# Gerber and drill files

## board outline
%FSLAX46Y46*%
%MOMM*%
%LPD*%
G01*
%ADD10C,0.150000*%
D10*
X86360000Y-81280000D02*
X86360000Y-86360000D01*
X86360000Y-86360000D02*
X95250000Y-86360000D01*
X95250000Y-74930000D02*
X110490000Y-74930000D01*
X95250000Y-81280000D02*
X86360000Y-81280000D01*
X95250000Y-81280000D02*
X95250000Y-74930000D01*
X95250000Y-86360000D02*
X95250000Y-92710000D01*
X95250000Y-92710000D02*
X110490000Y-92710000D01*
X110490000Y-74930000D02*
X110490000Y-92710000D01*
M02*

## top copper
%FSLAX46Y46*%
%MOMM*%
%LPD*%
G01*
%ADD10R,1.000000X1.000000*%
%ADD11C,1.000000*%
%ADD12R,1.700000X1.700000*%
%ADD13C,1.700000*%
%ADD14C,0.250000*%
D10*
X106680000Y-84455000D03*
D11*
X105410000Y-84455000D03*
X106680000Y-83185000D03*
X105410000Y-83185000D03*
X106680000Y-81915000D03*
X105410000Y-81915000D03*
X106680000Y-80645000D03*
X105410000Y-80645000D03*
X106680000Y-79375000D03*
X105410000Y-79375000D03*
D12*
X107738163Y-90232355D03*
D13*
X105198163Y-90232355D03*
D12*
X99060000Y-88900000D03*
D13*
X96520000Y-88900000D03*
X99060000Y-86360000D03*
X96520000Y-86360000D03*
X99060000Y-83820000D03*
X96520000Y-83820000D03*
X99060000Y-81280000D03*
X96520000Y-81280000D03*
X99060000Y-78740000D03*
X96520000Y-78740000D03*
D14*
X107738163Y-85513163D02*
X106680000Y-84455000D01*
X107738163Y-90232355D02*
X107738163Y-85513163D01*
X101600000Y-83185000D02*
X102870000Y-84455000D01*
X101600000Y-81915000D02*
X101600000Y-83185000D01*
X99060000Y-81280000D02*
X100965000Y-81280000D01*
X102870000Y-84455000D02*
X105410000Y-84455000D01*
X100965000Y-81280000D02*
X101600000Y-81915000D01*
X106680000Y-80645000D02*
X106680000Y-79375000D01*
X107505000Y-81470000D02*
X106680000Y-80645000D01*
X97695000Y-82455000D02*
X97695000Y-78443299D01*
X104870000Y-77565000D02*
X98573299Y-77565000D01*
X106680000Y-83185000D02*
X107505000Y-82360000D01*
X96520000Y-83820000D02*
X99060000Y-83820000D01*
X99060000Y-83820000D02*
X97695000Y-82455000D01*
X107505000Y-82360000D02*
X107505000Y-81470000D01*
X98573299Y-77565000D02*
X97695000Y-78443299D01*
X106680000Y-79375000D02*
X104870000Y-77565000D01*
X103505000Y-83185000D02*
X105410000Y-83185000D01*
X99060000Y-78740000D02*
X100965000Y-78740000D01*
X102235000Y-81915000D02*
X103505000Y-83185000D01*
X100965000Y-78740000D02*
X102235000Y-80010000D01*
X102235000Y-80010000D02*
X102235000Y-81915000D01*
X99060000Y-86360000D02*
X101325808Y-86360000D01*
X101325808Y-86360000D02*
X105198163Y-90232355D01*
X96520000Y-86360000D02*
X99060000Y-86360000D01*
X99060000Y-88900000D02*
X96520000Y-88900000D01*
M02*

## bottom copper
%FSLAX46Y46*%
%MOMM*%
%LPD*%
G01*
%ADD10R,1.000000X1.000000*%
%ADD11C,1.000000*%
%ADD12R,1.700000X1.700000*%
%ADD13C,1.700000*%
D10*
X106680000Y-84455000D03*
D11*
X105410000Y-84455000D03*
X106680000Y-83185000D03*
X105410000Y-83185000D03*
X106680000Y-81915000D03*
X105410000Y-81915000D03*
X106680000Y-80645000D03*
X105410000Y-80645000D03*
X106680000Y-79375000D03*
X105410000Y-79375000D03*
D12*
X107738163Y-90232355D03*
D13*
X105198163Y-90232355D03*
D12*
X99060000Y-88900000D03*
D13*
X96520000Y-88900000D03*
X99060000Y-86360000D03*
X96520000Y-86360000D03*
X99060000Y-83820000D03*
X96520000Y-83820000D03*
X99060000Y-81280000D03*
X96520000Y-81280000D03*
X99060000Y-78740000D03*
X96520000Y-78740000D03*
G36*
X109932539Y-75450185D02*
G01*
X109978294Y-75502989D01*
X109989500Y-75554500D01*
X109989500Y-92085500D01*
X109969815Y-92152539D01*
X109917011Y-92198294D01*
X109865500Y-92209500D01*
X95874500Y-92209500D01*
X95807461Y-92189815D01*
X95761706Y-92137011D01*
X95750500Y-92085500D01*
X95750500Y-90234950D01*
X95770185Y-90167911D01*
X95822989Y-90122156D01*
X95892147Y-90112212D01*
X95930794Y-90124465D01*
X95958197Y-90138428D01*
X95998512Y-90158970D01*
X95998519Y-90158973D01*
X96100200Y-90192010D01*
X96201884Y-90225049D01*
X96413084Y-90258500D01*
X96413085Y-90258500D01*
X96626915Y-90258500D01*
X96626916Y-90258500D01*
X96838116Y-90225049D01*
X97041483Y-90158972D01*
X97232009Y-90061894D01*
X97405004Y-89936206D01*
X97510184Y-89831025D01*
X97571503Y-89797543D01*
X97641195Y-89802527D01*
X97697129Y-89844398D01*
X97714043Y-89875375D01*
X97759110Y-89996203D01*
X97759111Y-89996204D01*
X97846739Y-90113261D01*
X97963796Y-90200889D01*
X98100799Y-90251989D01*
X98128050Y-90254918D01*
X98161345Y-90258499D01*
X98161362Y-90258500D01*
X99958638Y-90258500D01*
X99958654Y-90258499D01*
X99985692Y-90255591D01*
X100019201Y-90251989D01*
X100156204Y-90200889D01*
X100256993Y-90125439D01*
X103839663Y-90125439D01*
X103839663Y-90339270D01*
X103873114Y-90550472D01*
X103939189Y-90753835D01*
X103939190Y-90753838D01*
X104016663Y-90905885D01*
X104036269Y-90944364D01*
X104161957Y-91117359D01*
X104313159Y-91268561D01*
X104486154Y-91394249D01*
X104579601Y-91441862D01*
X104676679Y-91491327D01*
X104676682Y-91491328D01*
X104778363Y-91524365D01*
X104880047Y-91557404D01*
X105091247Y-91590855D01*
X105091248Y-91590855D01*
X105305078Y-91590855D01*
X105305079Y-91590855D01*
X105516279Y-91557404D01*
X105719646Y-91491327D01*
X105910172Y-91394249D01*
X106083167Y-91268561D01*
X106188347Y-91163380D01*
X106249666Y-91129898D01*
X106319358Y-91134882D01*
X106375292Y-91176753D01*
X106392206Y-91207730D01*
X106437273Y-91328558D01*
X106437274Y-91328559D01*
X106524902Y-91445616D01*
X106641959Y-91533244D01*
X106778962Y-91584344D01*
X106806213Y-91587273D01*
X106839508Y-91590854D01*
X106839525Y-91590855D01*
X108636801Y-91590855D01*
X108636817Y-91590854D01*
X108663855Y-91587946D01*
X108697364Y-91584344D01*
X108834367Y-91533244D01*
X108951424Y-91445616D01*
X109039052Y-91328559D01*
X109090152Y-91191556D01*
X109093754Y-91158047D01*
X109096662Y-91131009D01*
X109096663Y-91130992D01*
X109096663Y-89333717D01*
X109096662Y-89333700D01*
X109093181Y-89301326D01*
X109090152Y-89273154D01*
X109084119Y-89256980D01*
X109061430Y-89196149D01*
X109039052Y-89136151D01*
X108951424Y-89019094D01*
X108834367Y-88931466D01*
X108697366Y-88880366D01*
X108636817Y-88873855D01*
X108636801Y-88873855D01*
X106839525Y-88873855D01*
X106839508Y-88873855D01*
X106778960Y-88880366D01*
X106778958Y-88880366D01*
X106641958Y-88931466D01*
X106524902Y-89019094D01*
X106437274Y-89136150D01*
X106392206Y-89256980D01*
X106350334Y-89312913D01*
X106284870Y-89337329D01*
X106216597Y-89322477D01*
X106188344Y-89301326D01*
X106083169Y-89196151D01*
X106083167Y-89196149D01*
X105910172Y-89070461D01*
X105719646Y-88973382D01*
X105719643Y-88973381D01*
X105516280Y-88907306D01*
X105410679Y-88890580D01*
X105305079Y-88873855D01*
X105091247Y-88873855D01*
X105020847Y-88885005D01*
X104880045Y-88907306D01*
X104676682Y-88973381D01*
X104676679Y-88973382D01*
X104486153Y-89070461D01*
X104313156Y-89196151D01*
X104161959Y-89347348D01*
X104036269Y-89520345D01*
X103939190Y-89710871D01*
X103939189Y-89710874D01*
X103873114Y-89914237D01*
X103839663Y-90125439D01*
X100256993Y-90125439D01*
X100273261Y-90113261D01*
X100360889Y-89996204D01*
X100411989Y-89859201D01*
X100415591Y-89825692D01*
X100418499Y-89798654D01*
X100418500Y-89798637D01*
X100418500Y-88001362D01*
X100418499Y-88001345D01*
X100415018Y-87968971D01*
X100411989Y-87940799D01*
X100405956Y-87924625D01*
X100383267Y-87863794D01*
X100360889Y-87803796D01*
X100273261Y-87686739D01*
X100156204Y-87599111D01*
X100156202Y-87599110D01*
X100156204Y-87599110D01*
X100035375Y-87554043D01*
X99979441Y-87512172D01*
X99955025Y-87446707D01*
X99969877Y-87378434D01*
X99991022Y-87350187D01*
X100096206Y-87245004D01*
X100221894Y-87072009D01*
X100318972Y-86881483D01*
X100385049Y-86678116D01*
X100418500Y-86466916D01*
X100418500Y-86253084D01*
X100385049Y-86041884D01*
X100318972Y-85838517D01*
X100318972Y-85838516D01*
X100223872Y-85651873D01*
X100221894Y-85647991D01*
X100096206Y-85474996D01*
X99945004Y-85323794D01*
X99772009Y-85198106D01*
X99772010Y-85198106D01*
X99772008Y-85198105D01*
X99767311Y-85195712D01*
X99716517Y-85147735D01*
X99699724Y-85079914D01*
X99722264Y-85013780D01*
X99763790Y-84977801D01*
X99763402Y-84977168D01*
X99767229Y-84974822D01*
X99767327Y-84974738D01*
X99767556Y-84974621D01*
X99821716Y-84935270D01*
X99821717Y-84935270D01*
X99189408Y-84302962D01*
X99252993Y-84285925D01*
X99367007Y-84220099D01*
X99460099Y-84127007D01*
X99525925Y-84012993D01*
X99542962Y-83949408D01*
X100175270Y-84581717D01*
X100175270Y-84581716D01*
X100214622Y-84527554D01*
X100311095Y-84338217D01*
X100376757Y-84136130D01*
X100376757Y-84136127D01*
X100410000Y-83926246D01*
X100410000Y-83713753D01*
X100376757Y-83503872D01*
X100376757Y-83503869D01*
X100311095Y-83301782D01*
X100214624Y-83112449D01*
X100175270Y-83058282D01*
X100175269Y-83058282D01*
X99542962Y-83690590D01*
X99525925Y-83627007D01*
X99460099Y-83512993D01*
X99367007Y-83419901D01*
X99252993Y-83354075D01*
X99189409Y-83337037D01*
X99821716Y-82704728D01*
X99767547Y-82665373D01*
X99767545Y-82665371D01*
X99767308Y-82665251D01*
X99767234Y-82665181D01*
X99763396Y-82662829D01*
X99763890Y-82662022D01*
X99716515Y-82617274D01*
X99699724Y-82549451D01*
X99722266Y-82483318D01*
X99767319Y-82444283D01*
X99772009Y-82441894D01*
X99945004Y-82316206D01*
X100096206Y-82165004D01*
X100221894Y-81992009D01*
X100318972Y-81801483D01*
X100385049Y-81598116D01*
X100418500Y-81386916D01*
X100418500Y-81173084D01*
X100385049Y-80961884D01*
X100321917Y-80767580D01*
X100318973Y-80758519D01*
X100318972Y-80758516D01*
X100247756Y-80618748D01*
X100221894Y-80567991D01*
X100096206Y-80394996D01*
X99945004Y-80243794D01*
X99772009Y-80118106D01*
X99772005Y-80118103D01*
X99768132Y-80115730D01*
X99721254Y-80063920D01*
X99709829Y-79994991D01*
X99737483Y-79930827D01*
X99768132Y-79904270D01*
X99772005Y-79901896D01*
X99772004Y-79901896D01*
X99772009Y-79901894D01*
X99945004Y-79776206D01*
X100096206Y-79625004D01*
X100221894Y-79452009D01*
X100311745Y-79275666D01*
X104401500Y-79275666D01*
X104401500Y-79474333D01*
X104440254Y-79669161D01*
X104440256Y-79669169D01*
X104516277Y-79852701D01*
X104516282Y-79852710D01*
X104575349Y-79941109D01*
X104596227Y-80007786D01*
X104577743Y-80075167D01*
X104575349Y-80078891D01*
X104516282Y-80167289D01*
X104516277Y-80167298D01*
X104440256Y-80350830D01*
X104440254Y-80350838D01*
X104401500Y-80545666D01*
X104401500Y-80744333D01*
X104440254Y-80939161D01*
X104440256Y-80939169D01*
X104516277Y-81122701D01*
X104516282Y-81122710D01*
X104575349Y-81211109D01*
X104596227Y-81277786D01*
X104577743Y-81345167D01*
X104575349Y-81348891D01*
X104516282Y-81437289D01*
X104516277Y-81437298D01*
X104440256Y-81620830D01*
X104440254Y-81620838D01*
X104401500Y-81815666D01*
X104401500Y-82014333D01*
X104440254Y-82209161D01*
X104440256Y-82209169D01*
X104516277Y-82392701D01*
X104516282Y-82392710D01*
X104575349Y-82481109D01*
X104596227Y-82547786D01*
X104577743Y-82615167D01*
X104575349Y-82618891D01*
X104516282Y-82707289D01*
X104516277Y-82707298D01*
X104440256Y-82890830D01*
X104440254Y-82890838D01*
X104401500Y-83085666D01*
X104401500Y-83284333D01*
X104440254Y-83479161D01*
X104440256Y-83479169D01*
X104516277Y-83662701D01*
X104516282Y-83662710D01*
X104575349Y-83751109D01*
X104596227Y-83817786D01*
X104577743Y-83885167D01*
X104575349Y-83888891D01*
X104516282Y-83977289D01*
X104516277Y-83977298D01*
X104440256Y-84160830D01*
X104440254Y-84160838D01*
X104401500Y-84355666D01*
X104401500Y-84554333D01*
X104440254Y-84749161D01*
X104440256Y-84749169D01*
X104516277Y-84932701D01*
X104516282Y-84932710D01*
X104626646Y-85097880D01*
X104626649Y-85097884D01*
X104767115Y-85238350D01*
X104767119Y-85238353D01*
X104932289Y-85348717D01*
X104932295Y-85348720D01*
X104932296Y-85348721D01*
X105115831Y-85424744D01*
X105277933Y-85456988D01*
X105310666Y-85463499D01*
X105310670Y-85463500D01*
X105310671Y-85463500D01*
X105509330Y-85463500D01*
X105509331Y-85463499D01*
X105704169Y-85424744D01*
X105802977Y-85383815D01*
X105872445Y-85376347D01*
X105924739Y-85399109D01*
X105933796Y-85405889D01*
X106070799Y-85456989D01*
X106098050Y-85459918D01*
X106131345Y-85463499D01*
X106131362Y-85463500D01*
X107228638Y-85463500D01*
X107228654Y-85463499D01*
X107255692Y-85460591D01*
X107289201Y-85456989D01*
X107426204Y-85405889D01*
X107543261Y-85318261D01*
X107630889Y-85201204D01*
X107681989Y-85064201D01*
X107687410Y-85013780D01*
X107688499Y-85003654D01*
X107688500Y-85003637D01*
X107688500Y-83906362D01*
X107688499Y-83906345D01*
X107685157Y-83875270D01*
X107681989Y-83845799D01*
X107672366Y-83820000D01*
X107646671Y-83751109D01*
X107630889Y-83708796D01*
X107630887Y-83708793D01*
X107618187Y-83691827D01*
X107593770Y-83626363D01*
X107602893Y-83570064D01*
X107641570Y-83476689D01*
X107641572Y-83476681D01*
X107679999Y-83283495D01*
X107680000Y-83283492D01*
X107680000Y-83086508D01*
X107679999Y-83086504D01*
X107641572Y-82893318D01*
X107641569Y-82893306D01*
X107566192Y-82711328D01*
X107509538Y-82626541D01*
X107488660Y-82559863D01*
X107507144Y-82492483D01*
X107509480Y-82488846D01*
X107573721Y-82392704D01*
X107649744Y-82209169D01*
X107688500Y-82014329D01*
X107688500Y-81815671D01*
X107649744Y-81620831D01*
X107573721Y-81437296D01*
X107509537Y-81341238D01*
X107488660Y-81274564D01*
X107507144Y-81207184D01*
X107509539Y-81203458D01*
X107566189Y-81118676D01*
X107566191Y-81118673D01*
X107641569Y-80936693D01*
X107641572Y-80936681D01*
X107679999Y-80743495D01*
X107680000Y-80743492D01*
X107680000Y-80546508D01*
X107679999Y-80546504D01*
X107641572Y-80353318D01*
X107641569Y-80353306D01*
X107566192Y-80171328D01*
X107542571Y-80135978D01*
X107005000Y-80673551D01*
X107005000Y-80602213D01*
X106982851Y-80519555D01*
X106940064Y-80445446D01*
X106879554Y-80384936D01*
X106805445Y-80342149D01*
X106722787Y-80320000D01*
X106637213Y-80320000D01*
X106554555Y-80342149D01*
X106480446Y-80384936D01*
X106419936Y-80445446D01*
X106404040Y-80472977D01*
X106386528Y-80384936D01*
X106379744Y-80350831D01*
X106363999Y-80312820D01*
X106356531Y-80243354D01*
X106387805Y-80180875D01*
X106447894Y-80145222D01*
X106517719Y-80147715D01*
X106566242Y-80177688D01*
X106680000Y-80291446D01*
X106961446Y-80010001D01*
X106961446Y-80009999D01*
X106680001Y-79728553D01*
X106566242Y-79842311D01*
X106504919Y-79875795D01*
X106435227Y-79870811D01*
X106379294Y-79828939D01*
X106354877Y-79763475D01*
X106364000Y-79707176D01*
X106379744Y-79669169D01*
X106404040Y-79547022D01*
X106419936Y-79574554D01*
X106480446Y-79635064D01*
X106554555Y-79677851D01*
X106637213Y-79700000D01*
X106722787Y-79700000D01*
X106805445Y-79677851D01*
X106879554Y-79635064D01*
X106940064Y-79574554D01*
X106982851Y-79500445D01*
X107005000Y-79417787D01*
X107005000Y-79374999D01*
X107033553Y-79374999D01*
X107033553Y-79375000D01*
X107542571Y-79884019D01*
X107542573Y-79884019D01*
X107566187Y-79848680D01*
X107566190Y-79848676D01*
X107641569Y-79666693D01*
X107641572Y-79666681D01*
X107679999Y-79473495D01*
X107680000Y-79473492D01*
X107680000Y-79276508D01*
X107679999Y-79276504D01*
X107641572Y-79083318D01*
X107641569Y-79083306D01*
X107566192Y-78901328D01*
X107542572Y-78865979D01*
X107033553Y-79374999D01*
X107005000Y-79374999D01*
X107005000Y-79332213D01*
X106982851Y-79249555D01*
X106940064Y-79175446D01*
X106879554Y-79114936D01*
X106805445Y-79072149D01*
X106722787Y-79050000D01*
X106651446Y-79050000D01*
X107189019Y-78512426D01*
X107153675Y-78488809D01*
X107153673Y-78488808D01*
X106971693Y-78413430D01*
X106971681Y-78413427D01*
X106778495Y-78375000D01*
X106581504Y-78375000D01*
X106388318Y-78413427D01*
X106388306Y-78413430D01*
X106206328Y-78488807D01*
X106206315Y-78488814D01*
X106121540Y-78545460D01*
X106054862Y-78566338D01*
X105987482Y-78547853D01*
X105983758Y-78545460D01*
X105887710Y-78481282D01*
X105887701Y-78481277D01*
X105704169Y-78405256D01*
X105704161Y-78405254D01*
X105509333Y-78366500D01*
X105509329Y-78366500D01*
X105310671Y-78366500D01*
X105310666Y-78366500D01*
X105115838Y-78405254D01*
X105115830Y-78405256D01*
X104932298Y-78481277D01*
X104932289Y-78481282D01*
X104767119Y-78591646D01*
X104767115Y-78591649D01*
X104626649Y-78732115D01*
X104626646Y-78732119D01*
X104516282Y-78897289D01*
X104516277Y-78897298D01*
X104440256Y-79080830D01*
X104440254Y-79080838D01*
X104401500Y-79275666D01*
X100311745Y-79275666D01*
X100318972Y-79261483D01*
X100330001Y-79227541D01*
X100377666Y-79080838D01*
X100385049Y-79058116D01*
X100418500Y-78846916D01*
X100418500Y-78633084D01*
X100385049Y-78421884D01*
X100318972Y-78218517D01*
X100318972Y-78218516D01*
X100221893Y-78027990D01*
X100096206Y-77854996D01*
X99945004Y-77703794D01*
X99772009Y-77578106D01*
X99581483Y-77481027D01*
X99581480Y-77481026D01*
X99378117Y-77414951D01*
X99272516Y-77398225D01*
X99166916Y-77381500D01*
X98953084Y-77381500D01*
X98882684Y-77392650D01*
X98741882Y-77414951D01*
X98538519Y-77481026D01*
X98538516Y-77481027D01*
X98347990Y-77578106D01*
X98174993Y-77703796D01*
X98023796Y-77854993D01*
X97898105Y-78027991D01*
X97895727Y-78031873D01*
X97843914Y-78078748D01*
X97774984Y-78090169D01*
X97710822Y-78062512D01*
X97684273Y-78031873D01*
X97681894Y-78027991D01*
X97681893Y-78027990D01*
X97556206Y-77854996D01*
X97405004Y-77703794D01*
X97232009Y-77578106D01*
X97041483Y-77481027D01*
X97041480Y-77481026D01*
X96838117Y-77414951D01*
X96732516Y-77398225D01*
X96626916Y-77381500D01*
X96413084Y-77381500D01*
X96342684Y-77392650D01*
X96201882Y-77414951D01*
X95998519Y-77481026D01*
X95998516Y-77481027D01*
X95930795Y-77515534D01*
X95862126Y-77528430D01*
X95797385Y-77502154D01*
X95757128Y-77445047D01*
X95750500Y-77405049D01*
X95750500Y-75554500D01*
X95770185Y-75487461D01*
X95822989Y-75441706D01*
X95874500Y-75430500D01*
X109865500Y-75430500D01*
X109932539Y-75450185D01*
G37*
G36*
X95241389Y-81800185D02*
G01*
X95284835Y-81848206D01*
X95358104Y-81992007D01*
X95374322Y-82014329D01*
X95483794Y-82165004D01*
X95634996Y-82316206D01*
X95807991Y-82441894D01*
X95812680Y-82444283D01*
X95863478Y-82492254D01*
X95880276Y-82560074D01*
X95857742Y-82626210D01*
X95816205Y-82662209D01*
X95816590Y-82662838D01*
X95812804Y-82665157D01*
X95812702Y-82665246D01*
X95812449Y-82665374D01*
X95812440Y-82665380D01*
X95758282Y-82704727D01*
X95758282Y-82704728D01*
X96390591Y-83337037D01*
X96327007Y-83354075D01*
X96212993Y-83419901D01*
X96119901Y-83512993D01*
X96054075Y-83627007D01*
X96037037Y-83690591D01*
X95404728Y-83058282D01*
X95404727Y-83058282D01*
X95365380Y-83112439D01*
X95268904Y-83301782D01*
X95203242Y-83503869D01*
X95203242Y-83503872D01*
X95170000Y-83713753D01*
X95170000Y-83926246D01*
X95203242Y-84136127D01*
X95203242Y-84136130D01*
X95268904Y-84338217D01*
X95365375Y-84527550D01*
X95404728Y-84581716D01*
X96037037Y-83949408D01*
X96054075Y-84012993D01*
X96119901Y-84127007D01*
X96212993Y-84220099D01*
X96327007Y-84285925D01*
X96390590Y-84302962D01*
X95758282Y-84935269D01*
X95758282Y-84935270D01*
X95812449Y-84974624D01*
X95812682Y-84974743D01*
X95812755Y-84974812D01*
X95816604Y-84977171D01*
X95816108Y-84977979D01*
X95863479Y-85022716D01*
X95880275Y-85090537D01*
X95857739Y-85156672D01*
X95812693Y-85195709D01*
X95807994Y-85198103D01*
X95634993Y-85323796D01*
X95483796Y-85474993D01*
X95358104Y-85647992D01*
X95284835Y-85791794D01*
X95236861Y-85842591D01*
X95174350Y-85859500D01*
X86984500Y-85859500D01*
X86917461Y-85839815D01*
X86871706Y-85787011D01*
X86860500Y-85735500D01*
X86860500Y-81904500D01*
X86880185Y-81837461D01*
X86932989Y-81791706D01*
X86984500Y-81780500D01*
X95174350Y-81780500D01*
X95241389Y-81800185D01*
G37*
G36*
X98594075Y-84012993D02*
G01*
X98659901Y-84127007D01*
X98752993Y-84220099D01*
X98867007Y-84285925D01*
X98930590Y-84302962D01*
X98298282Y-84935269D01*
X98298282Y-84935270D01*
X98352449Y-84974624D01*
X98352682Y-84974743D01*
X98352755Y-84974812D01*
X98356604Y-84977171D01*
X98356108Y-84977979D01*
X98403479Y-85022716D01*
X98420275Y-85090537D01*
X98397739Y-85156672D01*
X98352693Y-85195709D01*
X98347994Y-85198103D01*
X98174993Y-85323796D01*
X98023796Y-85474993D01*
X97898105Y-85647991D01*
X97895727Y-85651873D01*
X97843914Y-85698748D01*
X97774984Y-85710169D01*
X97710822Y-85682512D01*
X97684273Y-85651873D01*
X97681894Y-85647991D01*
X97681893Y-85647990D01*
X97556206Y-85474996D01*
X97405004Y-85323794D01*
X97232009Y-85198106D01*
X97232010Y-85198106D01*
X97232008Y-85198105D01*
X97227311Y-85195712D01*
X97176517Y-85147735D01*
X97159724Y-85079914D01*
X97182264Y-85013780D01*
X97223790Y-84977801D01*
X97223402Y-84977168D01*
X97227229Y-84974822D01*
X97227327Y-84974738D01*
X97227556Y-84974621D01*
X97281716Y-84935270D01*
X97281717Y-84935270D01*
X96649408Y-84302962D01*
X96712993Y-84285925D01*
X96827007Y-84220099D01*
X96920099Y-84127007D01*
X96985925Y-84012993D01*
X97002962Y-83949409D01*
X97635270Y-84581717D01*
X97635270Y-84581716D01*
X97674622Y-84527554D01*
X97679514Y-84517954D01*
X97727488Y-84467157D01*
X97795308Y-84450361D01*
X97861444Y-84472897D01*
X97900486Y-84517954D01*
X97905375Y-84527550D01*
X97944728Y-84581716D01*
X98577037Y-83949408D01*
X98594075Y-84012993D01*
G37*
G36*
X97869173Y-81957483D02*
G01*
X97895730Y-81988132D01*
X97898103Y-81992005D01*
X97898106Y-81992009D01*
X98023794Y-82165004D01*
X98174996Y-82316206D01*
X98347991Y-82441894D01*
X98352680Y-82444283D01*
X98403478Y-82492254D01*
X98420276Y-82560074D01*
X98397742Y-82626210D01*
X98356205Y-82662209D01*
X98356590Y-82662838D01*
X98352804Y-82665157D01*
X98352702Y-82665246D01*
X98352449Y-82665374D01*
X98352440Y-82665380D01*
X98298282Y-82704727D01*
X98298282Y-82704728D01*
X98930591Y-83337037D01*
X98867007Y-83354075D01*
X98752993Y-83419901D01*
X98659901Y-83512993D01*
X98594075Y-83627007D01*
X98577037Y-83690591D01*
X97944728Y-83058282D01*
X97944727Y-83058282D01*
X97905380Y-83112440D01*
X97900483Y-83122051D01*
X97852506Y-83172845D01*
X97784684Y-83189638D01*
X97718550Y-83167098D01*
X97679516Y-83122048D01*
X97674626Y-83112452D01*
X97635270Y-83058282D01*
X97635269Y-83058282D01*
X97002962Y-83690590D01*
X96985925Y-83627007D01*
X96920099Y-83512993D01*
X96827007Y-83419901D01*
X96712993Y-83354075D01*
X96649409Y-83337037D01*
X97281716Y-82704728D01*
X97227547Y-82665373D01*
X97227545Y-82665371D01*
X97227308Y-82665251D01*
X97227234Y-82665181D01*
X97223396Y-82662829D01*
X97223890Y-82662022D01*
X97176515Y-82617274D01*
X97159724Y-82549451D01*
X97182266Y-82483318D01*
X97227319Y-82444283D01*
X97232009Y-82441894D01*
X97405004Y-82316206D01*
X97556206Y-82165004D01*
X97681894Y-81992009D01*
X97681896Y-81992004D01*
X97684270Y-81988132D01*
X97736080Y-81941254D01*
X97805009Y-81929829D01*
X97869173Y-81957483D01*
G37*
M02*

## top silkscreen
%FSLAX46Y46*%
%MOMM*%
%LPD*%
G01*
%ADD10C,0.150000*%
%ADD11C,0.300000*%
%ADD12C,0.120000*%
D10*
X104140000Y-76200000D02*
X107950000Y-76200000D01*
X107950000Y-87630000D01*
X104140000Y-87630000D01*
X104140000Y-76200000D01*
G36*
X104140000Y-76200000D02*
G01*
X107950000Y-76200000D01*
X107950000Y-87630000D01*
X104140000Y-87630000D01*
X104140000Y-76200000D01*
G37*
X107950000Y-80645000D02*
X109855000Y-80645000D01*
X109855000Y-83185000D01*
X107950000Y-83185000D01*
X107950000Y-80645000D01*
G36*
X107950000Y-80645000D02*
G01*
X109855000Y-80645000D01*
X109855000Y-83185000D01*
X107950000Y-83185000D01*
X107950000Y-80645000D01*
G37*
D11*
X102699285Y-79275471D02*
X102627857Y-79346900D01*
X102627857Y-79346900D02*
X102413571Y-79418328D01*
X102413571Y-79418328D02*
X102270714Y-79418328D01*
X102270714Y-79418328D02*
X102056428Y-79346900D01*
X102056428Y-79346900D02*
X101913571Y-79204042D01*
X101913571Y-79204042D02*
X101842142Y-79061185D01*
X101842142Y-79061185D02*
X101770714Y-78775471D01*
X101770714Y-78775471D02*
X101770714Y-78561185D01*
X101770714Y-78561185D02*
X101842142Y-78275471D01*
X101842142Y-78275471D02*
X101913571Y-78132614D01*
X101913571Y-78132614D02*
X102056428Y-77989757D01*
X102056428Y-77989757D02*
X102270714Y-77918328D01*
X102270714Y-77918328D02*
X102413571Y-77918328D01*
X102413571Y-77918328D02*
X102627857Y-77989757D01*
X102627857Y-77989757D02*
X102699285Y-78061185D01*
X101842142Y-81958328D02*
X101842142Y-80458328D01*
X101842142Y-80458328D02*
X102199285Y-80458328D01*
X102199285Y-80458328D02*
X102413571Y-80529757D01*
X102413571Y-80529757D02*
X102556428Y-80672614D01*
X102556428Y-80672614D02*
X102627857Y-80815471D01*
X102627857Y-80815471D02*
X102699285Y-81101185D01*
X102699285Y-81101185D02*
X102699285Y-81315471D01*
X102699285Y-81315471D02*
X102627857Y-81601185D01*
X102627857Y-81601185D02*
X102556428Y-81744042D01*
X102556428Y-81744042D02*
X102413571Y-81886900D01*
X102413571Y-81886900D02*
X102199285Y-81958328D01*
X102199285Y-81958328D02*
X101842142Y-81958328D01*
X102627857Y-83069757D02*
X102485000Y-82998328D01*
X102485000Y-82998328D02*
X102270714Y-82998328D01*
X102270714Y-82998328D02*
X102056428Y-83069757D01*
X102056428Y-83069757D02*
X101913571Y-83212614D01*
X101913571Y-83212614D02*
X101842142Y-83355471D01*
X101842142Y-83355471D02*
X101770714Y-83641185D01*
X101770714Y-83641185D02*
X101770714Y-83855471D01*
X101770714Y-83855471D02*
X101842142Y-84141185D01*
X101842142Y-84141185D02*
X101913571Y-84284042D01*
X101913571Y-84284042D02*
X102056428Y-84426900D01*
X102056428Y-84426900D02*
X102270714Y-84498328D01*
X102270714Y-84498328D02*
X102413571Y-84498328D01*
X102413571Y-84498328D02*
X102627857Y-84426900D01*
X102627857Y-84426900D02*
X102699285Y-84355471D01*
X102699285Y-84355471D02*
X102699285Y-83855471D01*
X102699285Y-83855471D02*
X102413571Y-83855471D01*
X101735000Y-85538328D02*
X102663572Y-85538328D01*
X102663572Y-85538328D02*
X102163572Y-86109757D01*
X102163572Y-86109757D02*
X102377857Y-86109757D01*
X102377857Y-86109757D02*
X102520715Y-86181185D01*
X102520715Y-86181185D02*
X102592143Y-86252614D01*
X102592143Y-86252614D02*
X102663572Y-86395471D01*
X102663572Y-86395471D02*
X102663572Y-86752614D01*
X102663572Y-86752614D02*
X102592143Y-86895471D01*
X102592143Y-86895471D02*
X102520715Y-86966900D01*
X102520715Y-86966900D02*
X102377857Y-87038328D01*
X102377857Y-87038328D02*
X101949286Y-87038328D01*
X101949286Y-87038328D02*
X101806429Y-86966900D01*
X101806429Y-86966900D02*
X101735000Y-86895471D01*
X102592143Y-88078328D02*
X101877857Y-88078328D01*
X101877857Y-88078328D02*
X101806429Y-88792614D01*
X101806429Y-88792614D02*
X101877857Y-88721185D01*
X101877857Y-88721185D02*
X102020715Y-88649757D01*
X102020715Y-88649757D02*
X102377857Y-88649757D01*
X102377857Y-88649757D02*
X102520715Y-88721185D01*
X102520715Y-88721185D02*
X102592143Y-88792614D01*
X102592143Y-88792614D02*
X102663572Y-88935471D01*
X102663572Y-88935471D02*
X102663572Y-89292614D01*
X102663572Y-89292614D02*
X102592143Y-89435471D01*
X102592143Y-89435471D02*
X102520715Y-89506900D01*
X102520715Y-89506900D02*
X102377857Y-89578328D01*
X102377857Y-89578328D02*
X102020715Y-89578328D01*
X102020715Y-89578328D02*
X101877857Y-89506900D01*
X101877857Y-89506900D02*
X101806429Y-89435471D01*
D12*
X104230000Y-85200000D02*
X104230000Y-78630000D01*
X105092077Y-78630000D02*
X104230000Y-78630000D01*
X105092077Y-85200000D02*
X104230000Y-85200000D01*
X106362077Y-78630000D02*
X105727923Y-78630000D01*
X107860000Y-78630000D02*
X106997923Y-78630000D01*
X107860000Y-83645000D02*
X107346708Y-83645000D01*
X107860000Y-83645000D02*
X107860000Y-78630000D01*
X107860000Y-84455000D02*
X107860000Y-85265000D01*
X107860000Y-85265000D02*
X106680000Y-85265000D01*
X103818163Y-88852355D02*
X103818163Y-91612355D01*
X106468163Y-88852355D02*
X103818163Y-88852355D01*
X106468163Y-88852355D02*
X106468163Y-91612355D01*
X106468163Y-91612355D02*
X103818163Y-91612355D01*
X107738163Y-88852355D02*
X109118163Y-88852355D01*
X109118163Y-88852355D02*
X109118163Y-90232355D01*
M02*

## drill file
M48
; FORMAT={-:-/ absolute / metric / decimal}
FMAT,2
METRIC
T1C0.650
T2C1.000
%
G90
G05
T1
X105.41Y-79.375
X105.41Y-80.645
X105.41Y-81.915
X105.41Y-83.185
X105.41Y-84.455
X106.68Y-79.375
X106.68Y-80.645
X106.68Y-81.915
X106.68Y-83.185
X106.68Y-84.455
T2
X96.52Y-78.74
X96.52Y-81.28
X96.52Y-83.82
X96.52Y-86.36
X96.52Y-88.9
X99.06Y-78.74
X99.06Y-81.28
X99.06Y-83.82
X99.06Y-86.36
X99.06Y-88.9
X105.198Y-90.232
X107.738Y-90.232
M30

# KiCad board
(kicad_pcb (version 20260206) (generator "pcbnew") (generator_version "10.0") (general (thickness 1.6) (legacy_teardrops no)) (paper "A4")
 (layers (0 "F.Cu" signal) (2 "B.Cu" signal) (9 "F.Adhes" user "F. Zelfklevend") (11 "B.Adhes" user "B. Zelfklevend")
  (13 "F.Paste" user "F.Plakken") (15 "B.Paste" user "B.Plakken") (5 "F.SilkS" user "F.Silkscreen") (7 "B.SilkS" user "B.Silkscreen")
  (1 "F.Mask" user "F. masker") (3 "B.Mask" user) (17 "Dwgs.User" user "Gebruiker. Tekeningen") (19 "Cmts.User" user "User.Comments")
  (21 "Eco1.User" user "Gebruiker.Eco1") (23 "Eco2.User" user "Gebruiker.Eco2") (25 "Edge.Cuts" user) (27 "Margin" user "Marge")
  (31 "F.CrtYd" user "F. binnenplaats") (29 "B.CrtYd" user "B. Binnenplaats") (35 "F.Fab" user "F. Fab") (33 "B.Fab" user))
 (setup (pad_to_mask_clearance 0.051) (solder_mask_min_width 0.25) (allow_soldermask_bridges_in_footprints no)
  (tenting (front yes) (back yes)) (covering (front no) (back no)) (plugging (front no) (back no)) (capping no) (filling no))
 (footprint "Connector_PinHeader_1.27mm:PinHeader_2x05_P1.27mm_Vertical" (layer "F.Cu") (at 106.68 84.455 180)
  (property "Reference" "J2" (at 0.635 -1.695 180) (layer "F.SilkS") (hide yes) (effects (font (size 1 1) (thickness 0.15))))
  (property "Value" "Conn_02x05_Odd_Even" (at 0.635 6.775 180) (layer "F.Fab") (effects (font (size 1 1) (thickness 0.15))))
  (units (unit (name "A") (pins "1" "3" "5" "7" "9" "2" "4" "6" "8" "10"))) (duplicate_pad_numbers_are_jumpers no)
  (fp_line (start 2.45 -0.745) (end 2.45 5.825) (stroke (width 0.12) (type solid)) (layer "F.SilkS"))
  (fp_line (start 1.587923 5.825) (end 2.45 5.825) (stroke (width 0.12) (type solid)) (layer "F.SilkS"))
  (fp_line (start 1.587923 -0.745) (end 2.45 -0.745) (stroke (width 0.12) (type solid)) (layer "F.SilkS"))
  (fp_line (start 0.317923 5.825) (end 0.952077 5.825) (stroke (width 0.12) (type solid)) (layer "F.SilkS"))
  (fp_line (start -1.18 5.825) (end -0.317923 5.825) (stroke (width 0.12) (type solid)) (layer "F.SilkS"))
  (fp_line (start -1.18 0.81) (end -0.666708 0.81) (stroke (width 0.12) (type solid)) (layer "F.SilkS"))
  (fp_line (start -1.18 0.81) (end -1.18 5.825) (stroke (width 0.12) (type solid)) (layer "F.SilkS"))
  (fp_line (start -1.18 0) (end -1.18 -0.81) (stroke (width 0.12) (type solid)) (layer "F.SilkS"))
  (fp_line (start -1.18 -0.81) (end 0 -0.81) (stroke (width 0.12) (type solid)) (layer "F.SilkS"))
  (pad "1" thru_hole rect (at 0 0 180) (size 1 1) (drill 0.65) (layers "*.Cu" "*.Mask") (remove_unused_layers no) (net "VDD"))
  (pad "2" thru_hole circle (at 1.27 0 180) (size 1 1) (drill 0.65) (layers "*.Cu" "*.Mask") (remove_unused_layers no) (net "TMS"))
  (pad "3" thru_hole circle (at 0 1.27 180) (size 1 1) (drill 0.65) (layers "*.Cu" "*.Mask") (remove_unused_layers no) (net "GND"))
  (pad "4" thru_hole circle (at 1.27 1.27 180) (size 1 1) (drill 0.65) (layers "*.Cu" "*.Mask") (remove_unused_layers no) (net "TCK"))
  (pad "5" thru_hole circle (at 0 2.54 180) (size 1 1) (drill 0.65) (layers "*.Cu" "*.Mask") (remove_unused_layers no)
   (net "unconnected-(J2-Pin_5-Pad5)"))
  (pad "6" thru_hole circle (at 1.27 2.54 180) (size 1 1) (drill 0.65) (layers "*.Cu" "*.Mask") (remove_unused_layers no) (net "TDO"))
  (pad "7" thru_hole circle (at 0 3.81 180) (size 1 1) (drill 0.65) (layers "*.Cu" "*.Mask") (remove_unused_layers no) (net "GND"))
  (pad "8" thru_hole circle (at 1.27 3.81 180) (size 1 1) (drill 0.65) (layers "*.Cu" "*.Mask") (remove_unused_layers no) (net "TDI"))
  (pad "9" thru_hole circle (at 0 5.08 180) (size 1 1) (drill 0.65) (layers "*.Cu" "*.Mask") (remove_unused_layers no) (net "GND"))
  (pad "10" thru_hole circle (at 1.27 5.08 180) (size 1 1) (drill 0.65) (layers "*.Cu" "*.Mask") (remove_unused_layers no) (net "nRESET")))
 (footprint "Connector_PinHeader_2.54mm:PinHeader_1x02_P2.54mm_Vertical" (layer "F.Cu") (at 107.738163 90.232355 -90)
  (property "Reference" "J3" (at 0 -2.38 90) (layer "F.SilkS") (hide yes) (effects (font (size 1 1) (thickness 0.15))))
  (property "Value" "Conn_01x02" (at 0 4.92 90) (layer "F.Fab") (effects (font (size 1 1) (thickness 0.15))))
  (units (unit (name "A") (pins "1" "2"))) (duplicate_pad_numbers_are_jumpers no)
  (fp_line (start -1.38 3.92) (end 1.38 3.92) (stroke (width 0.12) (type solid)) (layer "F.SilkS"))
  (fp_line (start -1.38 1.27) (end -1.38 3.92) (stroke (width 0.12) (type solid)) (layer "F.SilkS"))
  (fp_line (start -1.38 1.27) (end 1.38 1.27) (stroke (width 0.12) (type solid)) (layer "F.SilkS"))
  (fp_line (start 1.38 1.27) (end 1.38 3.92) (stroke (width 0.12) (type solid)) (layer "F.SilkS"))
  (fp_line (start -1.38 0) (end -1.38 -1.38) (stroke (width 0.12) (type solid)) (layer "F.SilkS"))
  (fp_line (start -1.38 -1.38) (end 0 -1.38) (stroke (width 0.12) (type solid)) (layer "F.SilkS"))
  (pad "1" thru_hole rect (at 0 0 270) (size 1.7 1.7) (drill 1) (layers "*.Cu" "*.Mask") (remove_unused_layers no) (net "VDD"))
  (pad "2" thru_hole circle (at 0 2.54 270) (size 1.7 1.7) (drill 1) (layers "*.Cu" "*.Mask") (remove_unused_layers no) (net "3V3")))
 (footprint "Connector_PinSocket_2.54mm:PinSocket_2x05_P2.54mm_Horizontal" (layer "B.Cu") (at 99.06 88.9)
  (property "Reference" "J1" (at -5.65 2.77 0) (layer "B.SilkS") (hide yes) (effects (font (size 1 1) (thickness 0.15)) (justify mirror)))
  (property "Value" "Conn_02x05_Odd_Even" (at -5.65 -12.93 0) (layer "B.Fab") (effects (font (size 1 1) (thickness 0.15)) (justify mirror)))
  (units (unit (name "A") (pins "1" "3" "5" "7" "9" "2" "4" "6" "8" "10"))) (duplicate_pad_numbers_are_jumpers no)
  (pad "1" thru_hole rect (at 0 0) (size 1.7 1.7) (drill 1) (layers "*.Cu" "*.Mask") (remove_unused_layers no) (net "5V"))
  (pad "2" thru_hole circle (at -2.54 0) (size 1.7 1.7) (drill 1) (layers "*.Cu" "*.Mask") (remove_unused_layers no) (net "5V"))
  (pad "3" thru_hole circle (at 0 -2.54) (size 1.7 1.7) (drill 1) (layers "*.Cu" "*.Mask") (remove_unused_layers no) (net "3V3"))
  (pad "4" thru_hole circle (at -2.54 -2.54) (size 1.7 1.7) (drill 1) (layers "*.Cu" "*.Mask") (remove_unused_layers no) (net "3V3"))
  (pad "5" thru_hole circle (at 0 -5.08) (size 1.7 1.7) (drill 1) (layers "*.Cu" "*.Mask") (remove_unused_layers no) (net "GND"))
  (pad "6" thru_hole circle (at -2.54 -5.08) (size 1.7 1.7) (drill 1) (layers "*.Cu" "*.Mask") (remove_unused_layers no) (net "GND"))
  (pad "7" thru_hole circle (at 0 -7.62) (size 1.7 1.7) (drill 1) (layers "*.Cu" "*.Mask") (remove_unused_layers no) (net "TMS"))
  (pad "8" thru_hole circle (at -2.54 -7.62) (size 1.7 1.7) (drill 1) (layers "*.Cu" "*.Mask") (remove_unused_layers no) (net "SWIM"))
  (pad "9" thru_hole circle (at 0 -10.16) (size 1.7 1.7) (drill 1) (layers "*.Cu" "*.Mask") (remove_unused_layers no) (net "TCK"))
  (pad "10" thru_hole circle (at -2.54 -10.16) (size 1.7 1.7) (drill 1) (layers "*.Cu" "*.Mask") (remove_unused_layers no)
   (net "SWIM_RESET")))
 (gr_rect (start 104.14 76.2) (end 107.95 87.63) (stroke (width 0.15) (type solid)) (fill yes) (layer "F.SilkS"))
 (gr_rect (start 107.95 80.645) (end 109.855 83.185) (stroke (width 0.15) (type solid)) (fill yes) (layer "F.SilkS"))
 (gr_line (start 86.36 81.28) (end 86.36 86.36) (stroke (width 0.15) (type default)) (layer "Edge.Cuts"))
 (gr_line (start 86.36 86.36) (end 95.25 86.36) (stroke (width 0.15) (type default)) (layer "Edge.Cuts"))
 (gr_line (start 95.25 74.93) (end 110.49 74.93) (stroke (width 0.15) (type default)) (layer "Edge.Cuts"))
 (gr_line (start 95.25 81.28) (end 86.36 81.28) (stroke (width 0.15) (type default)) (layer "Edge.Cuts"))
 (gr_line (start 95.25 81.28) (end 95.25 74.93) (stroke (width 0.15) (type default)) (layer "Edge.Cuts"))
 (gr_line (start 95.25 86.36) (end 95.25 92.71) (stroke (width 0.15) (type default)) (layer "Edge.Cuts"))
 (gr_line (start 95.25 92.71) (end 110.49 92.71) (stroke (width 0.15) (type default)) (layer "Edge.Cuts"))
 (gr_line (start 110.49 74.93) (end 110.49 92.71) (stroke (width 0.15) (type default)) (layer "Edge.Cuts"))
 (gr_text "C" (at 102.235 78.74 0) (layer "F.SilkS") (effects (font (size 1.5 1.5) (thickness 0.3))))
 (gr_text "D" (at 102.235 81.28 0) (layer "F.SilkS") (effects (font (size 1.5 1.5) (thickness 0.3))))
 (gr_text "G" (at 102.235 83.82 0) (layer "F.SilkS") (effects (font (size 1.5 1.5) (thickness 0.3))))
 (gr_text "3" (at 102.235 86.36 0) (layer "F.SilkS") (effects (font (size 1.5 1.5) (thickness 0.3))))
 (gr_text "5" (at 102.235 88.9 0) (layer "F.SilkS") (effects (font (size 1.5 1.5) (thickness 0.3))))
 (segment (start 107.738163 85.513163) (end 106.68 84.455) (width 0.25) (layer "F.Cu") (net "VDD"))
 (segment (start 107.738163 90.232355) (end 107.738163 85.513163) (width 0.25) (layer "F.Cu") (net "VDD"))
 (segment (start 101.6 83.185) (end 102.87 84.455) (width 0.25) (layer "F.Cu") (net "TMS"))
 (segment (start 101.6 81.915) (end 101.6 83.185) (width 0.25) (layer "F.Cu") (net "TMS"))
 (segment (start 99.06 81.28) (end 100.965 81.28) (width 0.25) (layer "F.Cu") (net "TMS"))
 (segment (start 102.87 84.455) (end 105.41 84.455) (width 0.25) (layer "F.Cu") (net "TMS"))
 (segment (start 100.965 81.28) (end 101.6 81.915) (width 0.25) (layer "F.Cu") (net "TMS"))
 (segment (start 106.68 80.645) (end 106.68 79.375) (width 0.25) (layer "F.Cu") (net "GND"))
 (segment (start 107.505 81.47) (end 106.68 80.645) (width 0.25) (layer "F.Cu") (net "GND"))
 (segment (start 97.695 82.455) (end 97.695 78.443299) (width 0.25) (layer "F.Cu") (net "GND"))
 (segment (start 104.87 77.565) (end 98.573299 77.565) (width 0.25) (layer "F.Cu") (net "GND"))
 (segment (start 106.68 83.185) (end 107.505 82.36) (width 0.25) (layer "F.Cu") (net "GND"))
 (segment (start 96.52 83.82) (end 99.06 83.82) (width 0.25) (layer "F.Cu") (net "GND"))
 (segment (start 99.06 83.82) (end 97.695 82.455) (width 0.25) (layer "F.Cu") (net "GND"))
 (segment (start 107.505 82.36) (end 107.505 81.47) (width 0.25) (layer "F.Cu") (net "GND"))
 (segment (start 98.573299 77.565) (end 97.695 78.443299) (width 0.25) (layer "F.Cu") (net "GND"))
 (segment (start 106.68 79.375) (end 104.87 77.565) (width 0.25) (layer "F.Cu") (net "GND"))
 (segment (start 103.505 83.185) (end 105.41 83.185) (width 0.25) (layer "F.Cu") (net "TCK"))
 (segment (start 99.06 78.74) (end 100.965 78.74) (width 0.25) (layer "F.Cu") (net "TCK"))
 (segment (start 102.235 81.915) (end 103.505 83.185) (width 0.25) (layer "F.Cu") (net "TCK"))
 (segment (start 100.965 78.74) (end 102.235 80.01) (width 0.25) (layer "F.Cu") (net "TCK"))
 (segment (start 102.235 80.01) (end 102.235 81.915) (width 0.25) (layer "F.Cu") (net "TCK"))
 (segment (start 99.06 86.36) (end 101.325808 86.36) (width 0.25) (layer "F.Cu") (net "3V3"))
 (segment (start 101.325808 86.36) (end 105.198163 90.232355) (width 0.25) (layer "F.Cu") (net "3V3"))
 (segment (start 96.52 86.36) (end 99.06 86.36) (width 0.25) (layer "F.Cu") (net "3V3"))
 (segment (start 99.06 88.9) (end 96.52 88.9) (width 0.25) (layer "F.Cu") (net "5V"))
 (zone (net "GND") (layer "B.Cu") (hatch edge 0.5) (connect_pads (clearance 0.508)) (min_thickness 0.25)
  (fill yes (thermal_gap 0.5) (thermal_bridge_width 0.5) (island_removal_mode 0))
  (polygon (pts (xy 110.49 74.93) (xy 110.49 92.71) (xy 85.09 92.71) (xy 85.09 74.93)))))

